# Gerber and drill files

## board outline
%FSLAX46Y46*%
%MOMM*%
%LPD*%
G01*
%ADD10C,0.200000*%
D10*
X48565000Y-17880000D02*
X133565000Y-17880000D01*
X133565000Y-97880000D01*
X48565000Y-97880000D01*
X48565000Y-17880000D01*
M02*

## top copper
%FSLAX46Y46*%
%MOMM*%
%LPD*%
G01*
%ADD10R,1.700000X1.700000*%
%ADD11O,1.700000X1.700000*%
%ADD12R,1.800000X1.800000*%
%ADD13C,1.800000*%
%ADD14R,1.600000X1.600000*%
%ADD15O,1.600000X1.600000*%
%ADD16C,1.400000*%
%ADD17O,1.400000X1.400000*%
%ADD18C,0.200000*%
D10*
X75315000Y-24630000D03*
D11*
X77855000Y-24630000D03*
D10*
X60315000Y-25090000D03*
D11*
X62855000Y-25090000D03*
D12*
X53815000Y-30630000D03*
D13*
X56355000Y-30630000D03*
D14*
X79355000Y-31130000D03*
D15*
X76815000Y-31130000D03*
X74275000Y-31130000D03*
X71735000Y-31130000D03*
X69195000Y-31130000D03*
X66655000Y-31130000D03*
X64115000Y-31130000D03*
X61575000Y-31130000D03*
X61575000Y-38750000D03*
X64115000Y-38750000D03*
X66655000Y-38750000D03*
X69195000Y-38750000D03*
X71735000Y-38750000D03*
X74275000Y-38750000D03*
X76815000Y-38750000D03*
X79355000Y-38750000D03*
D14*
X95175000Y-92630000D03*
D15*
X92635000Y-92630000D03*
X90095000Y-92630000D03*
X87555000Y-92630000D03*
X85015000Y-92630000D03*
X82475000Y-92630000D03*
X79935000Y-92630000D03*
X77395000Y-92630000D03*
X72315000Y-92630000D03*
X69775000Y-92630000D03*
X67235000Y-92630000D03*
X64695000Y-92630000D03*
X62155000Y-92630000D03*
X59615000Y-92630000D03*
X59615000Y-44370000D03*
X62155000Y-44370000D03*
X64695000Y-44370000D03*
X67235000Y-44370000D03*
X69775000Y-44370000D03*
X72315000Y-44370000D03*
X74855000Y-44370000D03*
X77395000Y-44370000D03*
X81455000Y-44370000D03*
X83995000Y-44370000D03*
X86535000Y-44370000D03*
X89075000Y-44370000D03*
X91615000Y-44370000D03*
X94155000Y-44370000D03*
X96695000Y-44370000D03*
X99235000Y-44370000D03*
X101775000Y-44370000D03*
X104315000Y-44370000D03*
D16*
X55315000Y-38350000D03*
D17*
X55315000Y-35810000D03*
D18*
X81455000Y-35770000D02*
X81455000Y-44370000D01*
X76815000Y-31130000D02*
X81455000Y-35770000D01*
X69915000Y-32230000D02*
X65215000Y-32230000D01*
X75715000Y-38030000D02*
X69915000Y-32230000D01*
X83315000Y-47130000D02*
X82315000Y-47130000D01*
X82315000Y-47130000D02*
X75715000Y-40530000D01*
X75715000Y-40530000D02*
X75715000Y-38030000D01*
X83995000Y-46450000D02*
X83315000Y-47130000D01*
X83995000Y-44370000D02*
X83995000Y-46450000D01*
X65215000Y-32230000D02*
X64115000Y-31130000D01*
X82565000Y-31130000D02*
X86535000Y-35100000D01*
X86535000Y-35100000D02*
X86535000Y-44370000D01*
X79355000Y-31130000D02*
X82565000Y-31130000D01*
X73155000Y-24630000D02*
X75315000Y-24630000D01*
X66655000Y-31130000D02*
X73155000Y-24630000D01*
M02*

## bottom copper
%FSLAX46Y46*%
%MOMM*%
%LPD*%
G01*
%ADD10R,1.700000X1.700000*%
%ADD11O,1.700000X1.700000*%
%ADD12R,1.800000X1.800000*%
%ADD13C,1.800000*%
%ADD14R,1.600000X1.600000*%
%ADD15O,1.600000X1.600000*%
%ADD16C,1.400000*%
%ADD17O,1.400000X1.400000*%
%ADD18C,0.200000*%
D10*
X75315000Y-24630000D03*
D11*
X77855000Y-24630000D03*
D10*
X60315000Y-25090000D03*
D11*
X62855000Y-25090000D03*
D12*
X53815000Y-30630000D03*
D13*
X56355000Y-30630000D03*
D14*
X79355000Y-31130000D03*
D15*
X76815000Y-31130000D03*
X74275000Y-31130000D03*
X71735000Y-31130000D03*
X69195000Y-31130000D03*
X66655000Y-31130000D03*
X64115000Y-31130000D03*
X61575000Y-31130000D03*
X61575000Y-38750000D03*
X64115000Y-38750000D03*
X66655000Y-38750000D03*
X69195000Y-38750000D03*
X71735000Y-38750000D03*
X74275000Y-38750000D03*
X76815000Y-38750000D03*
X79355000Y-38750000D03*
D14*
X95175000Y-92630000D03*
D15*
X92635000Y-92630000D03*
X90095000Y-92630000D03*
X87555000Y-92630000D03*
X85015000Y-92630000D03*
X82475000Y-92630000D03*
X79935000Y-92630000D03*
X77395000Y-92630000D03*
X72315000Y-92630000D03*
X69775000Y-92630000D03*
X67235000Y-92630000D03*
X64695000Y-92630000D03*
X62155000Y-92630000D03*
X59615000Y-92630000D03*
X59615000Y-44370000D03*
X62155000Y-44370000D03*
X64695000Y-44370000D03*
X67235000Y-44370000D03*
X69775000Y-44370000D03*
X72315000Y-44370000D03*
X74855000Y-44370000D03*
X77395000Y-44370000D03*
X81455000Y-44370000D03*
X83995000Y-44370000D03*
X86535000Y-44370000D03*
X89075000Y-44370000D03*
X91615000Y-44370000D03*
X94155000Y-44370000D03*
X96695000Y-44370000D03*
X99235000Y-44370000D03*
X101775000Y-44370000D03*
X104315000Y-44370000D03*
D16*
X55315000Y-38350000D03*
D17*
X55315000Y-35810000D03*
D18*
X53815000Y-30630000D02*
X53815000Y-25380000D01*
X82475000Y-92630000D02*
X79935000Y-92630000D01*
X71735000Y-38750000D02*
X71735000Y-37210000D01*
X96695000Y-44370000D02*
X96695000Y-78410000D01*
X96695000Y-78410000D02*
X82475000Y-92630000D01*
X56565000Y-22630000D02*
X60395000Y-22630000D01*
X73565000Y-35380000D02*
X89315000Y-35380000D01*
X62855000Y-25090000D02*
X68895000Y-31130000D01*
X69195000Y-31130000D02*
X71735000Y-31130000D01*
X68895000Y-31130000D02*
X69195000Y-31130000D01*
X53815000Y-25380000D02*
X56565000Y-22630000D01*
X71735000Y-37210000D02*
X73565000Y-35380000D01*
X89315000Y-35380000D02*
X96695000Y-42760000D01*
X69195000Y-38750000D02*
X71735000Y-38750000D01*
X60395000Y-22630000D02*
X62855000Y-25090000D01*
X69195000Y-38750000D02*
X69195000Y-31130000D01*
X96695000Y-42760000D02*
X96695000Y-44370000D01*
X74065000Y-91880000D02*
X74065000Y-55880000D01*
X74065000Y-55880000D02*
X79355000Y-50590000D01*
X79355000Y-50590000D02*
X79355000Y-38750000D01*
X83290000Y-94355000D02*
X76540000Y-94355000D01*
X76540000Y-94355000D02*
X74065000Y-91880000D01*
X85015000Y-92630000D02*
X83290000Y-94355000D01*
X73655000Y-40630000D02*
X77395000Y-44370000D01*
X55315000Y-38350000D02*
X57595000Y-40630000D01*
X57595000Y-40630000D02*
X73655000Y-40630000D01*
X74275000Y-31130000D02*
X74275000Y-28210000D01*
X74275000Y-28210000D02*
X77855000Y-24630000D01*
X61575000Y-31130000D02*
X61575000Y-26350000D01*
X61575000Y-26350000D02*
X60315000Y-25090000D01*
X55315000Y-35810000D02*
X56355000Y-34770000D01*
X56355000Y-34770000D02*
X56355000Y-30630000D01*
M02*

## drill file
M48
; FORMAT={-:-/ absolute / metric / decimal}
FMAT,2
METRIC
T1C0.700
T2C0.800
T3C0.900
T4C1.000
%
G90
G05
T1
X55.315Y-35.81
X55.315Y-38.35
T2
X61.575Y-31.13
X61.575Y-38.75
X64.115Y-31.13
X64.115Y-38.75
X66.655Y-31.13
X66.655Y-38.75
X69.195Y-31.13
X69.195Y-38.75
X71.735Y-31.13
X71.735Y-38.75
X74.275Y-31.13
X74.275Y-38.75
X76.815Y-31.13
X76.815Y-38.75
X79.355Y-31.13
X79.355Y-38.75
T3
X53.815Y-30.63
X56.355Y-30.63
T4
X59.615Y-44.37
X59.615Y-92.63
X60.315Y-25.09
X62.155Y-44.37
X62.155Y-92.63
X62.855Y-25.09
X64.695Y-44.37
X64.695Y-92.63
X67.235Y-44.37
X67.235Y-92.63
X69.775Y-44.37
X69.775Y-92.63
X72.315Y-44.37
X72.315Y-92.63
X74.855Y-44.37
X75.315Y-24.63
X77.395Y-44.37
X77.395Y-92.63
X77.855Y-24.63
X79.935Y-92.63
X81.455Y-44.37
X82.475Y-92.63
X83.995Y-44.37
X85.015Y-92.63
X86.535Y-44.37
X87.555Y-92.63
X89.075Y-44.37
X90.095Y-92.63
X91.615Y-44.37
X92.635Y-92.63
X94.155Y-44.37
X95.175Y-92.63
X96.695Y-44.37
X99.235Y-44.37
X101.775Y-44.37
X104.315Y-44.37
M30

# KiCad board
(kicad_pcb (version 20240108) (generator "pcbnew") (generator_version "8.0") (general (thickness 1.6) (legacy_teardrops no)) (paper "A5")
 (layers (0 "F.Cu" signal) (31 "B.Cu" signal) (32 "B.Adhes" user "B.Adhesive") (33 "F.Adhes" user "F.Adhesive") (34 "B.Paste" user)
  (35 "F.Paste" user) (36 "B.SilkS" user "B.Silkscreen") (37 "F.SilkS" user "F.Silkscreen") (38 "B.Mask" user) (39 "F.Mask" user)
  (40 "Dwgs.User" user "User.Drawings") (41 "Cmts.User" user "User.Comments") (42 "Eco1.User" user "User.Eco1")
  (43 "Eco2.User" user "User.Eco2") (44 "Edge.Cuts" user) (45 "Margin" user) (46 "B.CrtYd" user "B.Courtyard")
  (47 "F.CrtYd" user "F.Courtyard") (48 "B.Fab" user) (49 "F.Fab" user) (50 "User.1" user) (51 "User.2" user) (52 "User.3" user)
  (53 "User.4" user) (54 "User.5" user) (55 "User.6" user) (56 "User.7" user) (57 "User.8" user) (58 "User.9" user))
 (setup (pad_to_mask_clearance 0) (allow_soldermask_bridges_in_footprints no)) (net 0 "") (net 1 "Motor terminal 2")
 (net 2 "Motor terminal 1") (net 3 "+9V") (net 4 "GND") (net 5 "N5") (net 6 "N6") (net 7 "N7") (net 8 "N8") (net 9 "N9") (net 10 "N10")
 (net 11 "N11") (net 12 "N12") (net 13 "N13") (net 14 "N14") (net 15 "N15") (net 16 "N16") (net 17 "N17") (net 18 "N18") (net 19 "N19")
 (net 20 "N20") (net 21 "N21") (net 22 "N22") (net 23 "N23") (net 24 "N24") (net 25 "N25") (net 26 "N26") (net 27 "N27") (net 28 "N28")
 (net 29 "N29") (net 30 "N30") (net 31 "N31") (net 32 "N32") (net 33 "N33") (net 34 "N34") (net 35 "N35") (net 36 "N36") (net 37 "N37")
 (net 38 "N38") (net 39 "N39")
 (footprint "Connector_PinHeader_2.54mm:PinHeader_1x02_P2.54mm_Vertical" (layer "F.Cu") (at 75.315 24.63 90)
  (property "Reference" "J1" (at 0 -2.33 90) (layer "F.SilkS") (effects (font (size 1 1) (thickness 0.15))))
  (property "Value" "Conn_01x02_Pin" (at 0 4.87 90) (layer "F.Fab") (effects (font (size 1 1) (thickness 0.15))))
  (pad "1" thru_hole rect (at 0 0 90) (size 1.7 1.7) (drill 1) (layers "*.Cu" "*.Mask") (remove_unused_layers no) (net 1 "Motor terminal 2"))
  (pad "2" thru_hole oval (at 0 2.54 90) (size 1.7 1.7) (drill 1) (layers "*.Cu" "*.Mask") (remove_unused_layers no)
   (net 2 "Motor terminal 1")))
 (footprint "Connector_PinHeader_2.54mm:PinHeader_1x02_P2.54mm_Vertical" (layer "F.Cu") (at 60.315 25.09 90)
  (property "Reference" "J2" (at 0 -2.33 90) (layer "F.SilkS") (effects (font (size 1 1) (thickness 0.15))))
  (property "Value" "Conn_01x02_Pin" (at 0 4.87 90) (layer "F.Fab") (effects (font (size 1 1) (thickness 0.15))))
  (pad "1" thru_hole rect (at 0 0 90) (size 1.7 1.7) (drill 1) (layers "*.Cu" "*.Mask") (remove_unused_layers no) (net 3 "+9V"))
  (pad "2" thru_hole oval (at 0 2.54 90) (size 1.7 1.7) (drill 1) (layers "*.Cu" "*.Mask") (remove_unused_layers no) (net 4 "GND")))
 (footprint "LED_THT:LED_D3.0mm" (layer "F.Cu") (at 53.815 30.63)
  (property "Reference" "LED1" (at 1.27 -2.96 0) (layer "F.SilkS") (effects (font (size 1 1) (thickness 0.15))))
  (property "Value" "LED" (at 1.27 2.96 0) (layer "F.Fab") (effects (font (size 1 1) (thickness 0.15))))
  (pad "1" thru_hole rect (at 0 0) (size 1.8 1.8) (drill 0.9) (layers "*.Cu" "*.Mask") (remove_unused_layers no) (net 4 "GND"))
  (pad "2" thru_hole circle (at 2.54 0) (size 1.8 1.8) (drill 0.9) (layers "*.Cu" "*.Mask") (remove_unused_layers no) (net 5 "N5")))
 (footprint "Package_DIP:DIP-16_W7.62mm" (layer "F.Cu") (at 79.355 31.13 -90)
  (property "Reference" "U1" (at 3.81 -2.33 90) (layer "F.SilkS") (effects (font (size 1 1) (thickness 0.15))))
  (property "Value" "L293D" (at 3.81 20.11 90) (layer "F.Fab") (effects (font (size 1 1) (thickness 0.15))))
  (pad "1" thru_hole rect (at 0 0 270) (size 1.6 1.6) (drill 0.8) (layers "*.Cu" "*.Mask") (remove_unused_layers no) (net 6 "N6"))
  (pad "2" thru_hole oval (at 0 2.54 270) (size 1.6 1.6) (drill 0.8) (layers "*.Cu" "*.Mask") (remove_unused_layers no) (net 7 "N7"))
  (pad "3" thru_hole oval (at 0 5.08 270) (size 1.6 1.6) (drill 0.8) (layers "*.Cu" "*.Mask") (remove_unused_layers no)
   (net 2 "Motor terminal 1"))
  (pad "4" thru_hole oval (at 0 7.62 270) (size 1.6 1.6) (drill 0.8) (layers "*.Cu" "*.Mask") (remove_unused_layers no) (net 4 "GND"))
  (pad "5" thru_hole oval (at 0 10.16 270) (size 1.6 1.6) (drill 0.8) (layers "*.Cu" "*.Mask") (remove_unused_layers no) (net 4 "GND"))
  (pad "6" thru_hole oval (at 0 12.7 270) (size 1.6 1.6) (drill 0.8) (layers "*.Cu" "*.Mask") (remove_unused_layers no)
   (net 1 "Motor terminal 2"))
  (pad "7" thru_hole oval (at 0 15.24 270) (size 1.6 1.6) (drill 0.8) (layers "*.Cu" "*.Mask") (remove_unused_layers no) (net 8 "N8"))
  (pad "8" thru_hole oval (at 0 17.78 270) (size 1.6 1.6) (drill 0.8) (layers "*.Cu" "*.Mask") (remove_unused_layers no) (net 3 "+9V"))
  (pad "9" thru_hole oval (at 7.62 17.78 270) (size 1.6 1.6) (drill 0.8) (layers "*.Cu" "*.Mask") (remove_unused_layers no) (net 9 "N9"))
  (pad "10" thru_hole oval (at 7.62 15.24 270) (size 1.6 1.6) (drill 0.8) (layers "*.Cu" "*.Mask") (remove_unused_layers no) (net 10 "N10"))
  (pad "11" thru_hole oval (at 7.62 12.7 270) (size 1.6 1.6) (drill 0.8) (layers "*.Cu" "*.Mask") (remove_unused_layers no) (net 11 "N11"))
  (pad "12" thru_hole oval (at 7.62 10.16 270) (size 1.6 1.6) (drill 0.8) (layers "*.Cu" "*.Mask") (remove_unused_layers no) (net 4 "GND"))
  (pad "13" thru_hole oval (at 7.62 7.62 270) (size 1.6 1.6) (drill 0.8) (layers "*.Cu" "*.Mask") (remove_unused_layers no) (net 4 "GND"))
  (pad "14" thru_hole oval (at 7.62 5.08 270) (size 1.6 1.6) (drill 0.8) (layers "*.Cu" "*.Mask") (remove_unused_layers no) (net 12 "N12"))
  (pad "15" thru_hole oval (at 7.62 2.54 270) (size 1.6 1.6) (drill 0.8) (layers "*.Cu" "*.Mask") (remove_unused_layers no) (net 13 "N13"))
  (pad "16" thru_hole oval (at 7.62 0 270) (size 1.6 1.6) (drill 0.8) (layers "*.Cu" "*.Mask") (remove_unused_layers no) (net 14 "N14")))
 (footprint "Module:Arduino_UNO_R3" (layer "F.Cu") (at 95.175 92.63 180)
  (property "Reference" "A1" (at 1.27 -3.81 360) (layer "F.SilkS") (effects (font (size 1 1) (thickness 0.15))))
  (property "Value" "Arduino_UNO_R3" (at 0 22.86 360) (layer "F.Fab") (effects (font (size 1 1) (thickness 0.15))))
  (pad "1" thru_hole rect (at 0 0 270) (size 1.6 1.6) (drill 1) (layers "*.Cu" "*.Mask") (remove_unused_layers no) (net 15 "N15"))
  (pad "2" thru_hole oval (at 2.54 0 270) (size 1.6 1.6) (drill 1) (layers "*.Cu" "*.Mask") (remove_unused_layers no) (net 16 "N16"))
  (pad "3" thru_hole oval (at 5.08 0 270) (size 1.6 1.6) (drill 1) (layers "*.Cu" "*.Mask") (remove_unused_layers no) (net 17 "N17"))
  (pad "4" thru_hole oval (at 7.62 0 270) (size 1.6 1.6) (drill 1) (layers "*.Cu" "*.Mask") (remove_unused_layers no) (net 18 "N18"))
  (pad "5" thru_hole oval (at 10.16 0 270) (size 1.6 1.6) (drill 1) (layers "*.Cu" "*.Mask") (remove_unused_layers no) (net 14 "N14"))
  (pad "6" thru_hole oval (at 12.7 0 270) (size 1.6 1.6) (drill 1) (layers "*.Cu" "*.Mask") (remove_unused_layers no) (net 4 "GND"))
  (pad "7" thru_hole oval (at 15.24 0 270) (size 1.6 1.6) (drill 1) (layers "*.Cu" "*.Mask") (remove_unused_layers no) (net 4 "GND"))
  (pad "8" thru_hole oval (at 17.78 0 270) (size 1.6 1.6) (drill 1) (layers "*.Cu" "*.Mask") (remove_unused_layers no) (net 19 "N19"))
  (pad "9" thru_hole oval (at 22.86 0 270) (size 1.6 1.6) (drill 1) (layers "*.Cu" "*.Mask") (remove_unused_layers no) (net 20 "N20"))
  (pad "10" thru_hole oval (at 25.4 0 270) (size 1.6 1.6) (drill 1) (layers "*.Cu" "*.Mask") (remove_unused_layers no) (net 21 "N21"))
  (pad "11" thru_hole oval (at 27.94 0 270) (size 1.6 1.6) (drill 1) (layers "*.Cu" "*.Mask") (remove_unused_layers no) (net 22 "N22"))
  (pad "12" thru_hole oval (at 30.48 0 270) (size 1.6 1.6) (drill 1) (layers "*.Cu" "*.Mask") (remove_unused_layers no) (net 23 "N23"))
  (pad "13" thru_hole oval (at 33.02 0 270) (size 1.6 1.6) (drill 1) (layers "*.Cu" "*.Mask") (remove_unused_layers no) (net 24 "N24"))
  (pad "14" thru_hole oval (at 35.56 0 270) (size 1.6 1.6) (drill 1) (layers "*.Cu" "*.Mask") (remove_unused_layers no) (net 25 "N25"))
  (pad "15" thru_hole oval (at 35.56 48.26 270) (size 1.6 1.6) (drill 1) (layers "*.Cu" "*.Mask") (remove_unused_layers no) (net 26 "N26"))
  (pad "16" thru_hole oval (at 33.02 48.26 270) (size 1.6 1.6) (drill 1) (layers "*.Cu" "*.Mask") (remove_unused_layers no) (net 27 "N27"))
  (pad "17" thru_hole oval (at 30.48 48.26 270) (size 1.6 1.6) (drill 1) (layers "*.Cu" "*.Mask") (remove_unused_layers no) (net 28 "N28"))
  (pad "18" thru_hole oval (at 27.94 48.26 270) (size 1.6 1.6) (drill 1) (layers "*.Cu" "*.Mask") (remove_unused_layers no) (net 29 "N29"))
  (pad "19" thru_hole oval (at 25.4 48.26 270) (size 1.6 1.6) (drill 1) (layers "*.Cu" "*.Mask") (remove_unused_layers no) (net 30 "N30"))
  (pad "20" thru_hole oval (at 22.86 48.26 270) (size 1.6 1.6) (drill 1) (layers "*.Cu" "*.Mask") (remove_unused_layers no) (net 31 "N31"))
  (pad "21" thru_hole oval (at 20.32 48.26 270) (size 1.6 1.6) (drill 1) (layers "*.Cu" "*.Mask") (remove_unused_layers no) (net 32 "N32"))
  (pad "22" thru_hole oval (at 17.78 48.26 270) (size 1.6 1.6) (drill 1) (layers "*.Cu" "*.Mask") (remove_unused_layers no) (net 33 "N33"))
  (pad "23" thru_hole oval (at 13.72 48.26 270) (size 1.6 1.6) (drill 1) (layers "*.Cu" "*.Mask") (remove_unused_layers no) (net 7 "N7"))
  (pad "24" thru_hole oval (at 11.18 48.26 270) (size 1.6 1.6) (drill 1) (layers "*.Cu" "*.Mask") (remove_unused_layers no) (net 8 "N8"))
  (pad "25" thru_hole oval (at 8.64 48.26 270) (size 1.6 1.6) (drill 1) (layers "*.Cu" "*.Mask") (remove_unused_layers no) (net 6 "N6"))
  (pad "26" thru_hole oval (at 6.1 48.26 270) (size 1.6 1.6) (drill 1) (layers "*.Cu" "*.Mask") (remove_unused_layers no) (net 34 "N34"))
  (pad "27" thru_hole oval (at 3.56 48.26 270) (size 1.6 1.6) (drill 1) (layers "*.Cu" "*.Mask") (remove_unused_layers no) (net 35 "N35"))
  (pad "28" thru_hole oval (at 1.02 48.26 270) (size 1.6 1.6) (drill 1) (layers "*.Cu" "*.Mask") (remove_unused_layers no) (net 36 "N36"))
  (pad "29" thru_hole oval (at -1.52 48.26 270) (size 1.6 1.6) (drill 1) (layers "*.Cu" "*.Mask") (remove_unused_layers no) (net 4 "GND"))
  (pad "30" thru_hole oval (at -4.06 48.26 270) (size 1.6 1.6) (drill 1) (layers "*.Cu" "*.Mask") (remove_unused_layers no) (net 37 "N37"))
  (pad "31" thru_hole oval (at -6.6 48.26 270) (size 1.6 1.6) (drill 1) (layers "*.Cu" "*.Mask") (remove_unused_layers no) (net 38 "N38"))
  (pad "32" thru_hole oval (at -9.14 48.26 270) (size 1.6 1.6) (drill 1) (layers "*.Cu" "*.Mask") (remove_unused_layers no) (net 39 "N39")))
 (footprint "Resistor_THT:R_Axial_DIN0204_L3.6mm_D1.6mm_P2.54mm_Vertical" (layer "F.Cu") (at 55.315 38.35 90)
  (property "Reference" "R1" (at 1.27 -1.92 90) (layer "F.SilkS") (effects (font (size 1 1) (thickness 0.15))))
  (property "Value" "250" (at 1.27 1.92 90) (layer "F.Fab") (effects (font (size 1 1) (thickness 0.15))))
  (pad "1" thru_hole circle (at 0 0 90) (size 1.4 1.4) (drill 0.7) (layers "*.Cu" "*.Mask") (remove_unused_layers no) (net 33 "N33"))
  (pad "2" thru_hole oval (at 2.54 0 90) (size 1.4 1.4) (drill 0.7) (layers "*.Cu" "*.Mask") (remove_unused_layers no) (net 5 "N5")))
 (gr_rect (start 48.565 17.88) (end 133.565 97.88) (stroke (width 0.2) (type default)) (fill none) (layer "Edge.Cuts"))
 (segment (start 81.455 35.77) (end 81.455 44.37) (width 0.2) (layer "F.Cu") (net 7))
 (segment (start 76.815 31.13) (end 81.455 35.77) (width 0.2) (layer "F.Cu") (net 7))
 (segment (start 53.815 30.63) (end 53.815 25.38) (width 0.2) (layer "B.Cu") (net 4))
 (segment (start 82.475 92.63) (end 79.935 92.63) (width 0.2) (layer "B.Cu") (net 4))
 (segment (start 71.735 38.75) (end 71.735 37.21) (width 0.2) (layer "B.Cu") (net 4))
 (segment (start 96.695 44.37) (end 96.695 78.41) (width 0.2) (layer "B.Cu") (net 4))
 (segment (start 96.695 78.41) (end 82.475 92.63) (width 0.2) (layer "B.Cu") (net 4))
 (segment (start 56.565 22.63) (end 60.395 22.63) (width 0.2) (layer "B.Cu") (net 4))
 (segment (start 73.565 35.38) (end 89.315 35.38) (width 0.2) (layer "B.Cu") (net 4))
 (segment (start 62.855 25.09) (end 68.895 31.13) (width 0.2) (layer "B.Cu") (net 4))
 (segment (start 69.195 31.13) (end 71.735 31.13) (width 0.2) (layer "B.Cu") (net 4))
 (segment (start 68.895 31.13) (end 69.195 31.13) (width 0.2) (layer "B.Cu") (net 4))
 (segment (start 53.815 25.38) (end 56.565 22.63) (width 0.2) (layer "B.Cu") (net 4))
 (segment (start 71.735 37.21) (end 73.565 35.38) (width 0.2) (layer "B.Cu") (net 4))
 (segment (start 89.315 35.38) (end 96.695 42.76) (width 0.2) (layer "B.Cu") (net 4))
 (segment (start 69.195 38.75) (end 71.735 38.75) (width 0.2) (layer "B.Cu") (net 4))
 (segment (start 60.395 22.63) (end 62.855 25.09) (width 0.2) (layer "B.Cu") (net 4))
 (segment (start 69.195 38.75) (end 69.195 31.13) (width 0.2) (layer "B.Cu") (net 4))
 (segment (start 96.695 42.76) (end 96.695 44.37) (width 0.2) (layer "B.Cu") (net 4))
 (segment (start 74.065 91.88) (end 74.065 55.88) (width 0.2) (layer "B.Cu") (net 14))
 (segment (start 74.065 55.88) (end 79.355 50.59) (width 0.2) (layer "B.Cu") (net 14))
 (segment (start 79.355 50.59) (end 79.355 38.75) (width 0.2) (layer "B.Cu") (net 14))
 (segment (start 83.29 94.355) (end 76.54 94.355) (width 0.2) (layer "B.Cu") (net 14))
 (segment (start 76.54 94.355) (end 74.065 91.88) (width 0.2) (layer "B.Cu") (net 14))
 (segment (start 85.015 92.63) (end 83.29 94.355) (width 0.2) (layer "B.Cu") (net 14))
 (segment (start 69.915 32.23) (end 65.215 32.23) (width 0.2) (layer "F.Cu") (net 8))
 (segment (start 75.715 38.03) (end 69.915 32.23) (width 0.2) (layer "F.Cu") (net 8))
 (segment (start 83.315 47.13) (end 82.315 47.13) (width 0.2) (layer "F.Cu") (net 8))
 (segment (start 82.315 47.13) (end 75.715 40.53) (width 0.2) (layer "F.Cu") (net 8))
 (segment (start 75.715 40.53) (end 75.715 38.03) (width 0.2) (layer "F.Cu") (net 8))
 (segment (start 83.995 46.45) (end 83.315 47.13) (width 0.2) (layer "F.Cu") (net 8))
 (segment (start 83.995 44.37) (end 83.995 46.45) (width 0.2) (layer "F.Cu") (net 8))
 (segment (start 65.215 32.23) (end 64.115 31.13) (width 0.2) (layer "F.Cu") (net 8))
 (segment (start 82.565 31.13) (end 86.535 35.1) (width 0.2) (layer "F.Cu") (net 6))
 (segment (start 86.535 35.1) (end 86.535 44.37) (width 0.2) (layer "F.Cu") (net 6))
 (segment (start 79.355 31.13) (end 82.565 31.13) (width 0.2) (layer "F.Cu") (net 6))
 (segment (start 73.655 40.63) (end 77.395 44.37) (width 0.2) (layer "B.Cu") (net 33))
 (segment (start 55.315 38.35) (end 57.595 40.63) (width 0.2) (layer "B.Cu") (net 33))
 (segment (start 57.595 40.63) (end 73.655 40.63) (width 0.2) (layer "B.Cu") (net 33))
 (segment (start 74.275 31.13) (end 74.275 28.21) (width 0.2) (layer "B.Cu") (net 2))
 (segment (start 74.275 28.21) (end 77.855 24.63) (width 0.2) (layer "B.Cu") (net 2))
 (segment (start 73.155 24.63) (end 75.315 24.63) (width 0.2) (layer "F.Cu") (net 1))
 (segment (start 66.655 31.13) (end 73.155 24.63) (width 0.2) (layer "F.Cu") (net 1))
 (segment (start 61.575 31.13) (end 61.575 26.35) (width 0.2) (layer "B.Cu") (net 3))
 (segment (start 61.575 26.35) (end 60.315 25.09) (width 0.2) (layer "B.Cu") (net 3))
 (segment (start 55.315 35.81) (end 56.355 34.77) (width 0.2) (layer "B.Cu") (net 5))
 (segment (start 56.355 34.77) (end 56.355 30.63) (width 0.2) (layer "B.Cu") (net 5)))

